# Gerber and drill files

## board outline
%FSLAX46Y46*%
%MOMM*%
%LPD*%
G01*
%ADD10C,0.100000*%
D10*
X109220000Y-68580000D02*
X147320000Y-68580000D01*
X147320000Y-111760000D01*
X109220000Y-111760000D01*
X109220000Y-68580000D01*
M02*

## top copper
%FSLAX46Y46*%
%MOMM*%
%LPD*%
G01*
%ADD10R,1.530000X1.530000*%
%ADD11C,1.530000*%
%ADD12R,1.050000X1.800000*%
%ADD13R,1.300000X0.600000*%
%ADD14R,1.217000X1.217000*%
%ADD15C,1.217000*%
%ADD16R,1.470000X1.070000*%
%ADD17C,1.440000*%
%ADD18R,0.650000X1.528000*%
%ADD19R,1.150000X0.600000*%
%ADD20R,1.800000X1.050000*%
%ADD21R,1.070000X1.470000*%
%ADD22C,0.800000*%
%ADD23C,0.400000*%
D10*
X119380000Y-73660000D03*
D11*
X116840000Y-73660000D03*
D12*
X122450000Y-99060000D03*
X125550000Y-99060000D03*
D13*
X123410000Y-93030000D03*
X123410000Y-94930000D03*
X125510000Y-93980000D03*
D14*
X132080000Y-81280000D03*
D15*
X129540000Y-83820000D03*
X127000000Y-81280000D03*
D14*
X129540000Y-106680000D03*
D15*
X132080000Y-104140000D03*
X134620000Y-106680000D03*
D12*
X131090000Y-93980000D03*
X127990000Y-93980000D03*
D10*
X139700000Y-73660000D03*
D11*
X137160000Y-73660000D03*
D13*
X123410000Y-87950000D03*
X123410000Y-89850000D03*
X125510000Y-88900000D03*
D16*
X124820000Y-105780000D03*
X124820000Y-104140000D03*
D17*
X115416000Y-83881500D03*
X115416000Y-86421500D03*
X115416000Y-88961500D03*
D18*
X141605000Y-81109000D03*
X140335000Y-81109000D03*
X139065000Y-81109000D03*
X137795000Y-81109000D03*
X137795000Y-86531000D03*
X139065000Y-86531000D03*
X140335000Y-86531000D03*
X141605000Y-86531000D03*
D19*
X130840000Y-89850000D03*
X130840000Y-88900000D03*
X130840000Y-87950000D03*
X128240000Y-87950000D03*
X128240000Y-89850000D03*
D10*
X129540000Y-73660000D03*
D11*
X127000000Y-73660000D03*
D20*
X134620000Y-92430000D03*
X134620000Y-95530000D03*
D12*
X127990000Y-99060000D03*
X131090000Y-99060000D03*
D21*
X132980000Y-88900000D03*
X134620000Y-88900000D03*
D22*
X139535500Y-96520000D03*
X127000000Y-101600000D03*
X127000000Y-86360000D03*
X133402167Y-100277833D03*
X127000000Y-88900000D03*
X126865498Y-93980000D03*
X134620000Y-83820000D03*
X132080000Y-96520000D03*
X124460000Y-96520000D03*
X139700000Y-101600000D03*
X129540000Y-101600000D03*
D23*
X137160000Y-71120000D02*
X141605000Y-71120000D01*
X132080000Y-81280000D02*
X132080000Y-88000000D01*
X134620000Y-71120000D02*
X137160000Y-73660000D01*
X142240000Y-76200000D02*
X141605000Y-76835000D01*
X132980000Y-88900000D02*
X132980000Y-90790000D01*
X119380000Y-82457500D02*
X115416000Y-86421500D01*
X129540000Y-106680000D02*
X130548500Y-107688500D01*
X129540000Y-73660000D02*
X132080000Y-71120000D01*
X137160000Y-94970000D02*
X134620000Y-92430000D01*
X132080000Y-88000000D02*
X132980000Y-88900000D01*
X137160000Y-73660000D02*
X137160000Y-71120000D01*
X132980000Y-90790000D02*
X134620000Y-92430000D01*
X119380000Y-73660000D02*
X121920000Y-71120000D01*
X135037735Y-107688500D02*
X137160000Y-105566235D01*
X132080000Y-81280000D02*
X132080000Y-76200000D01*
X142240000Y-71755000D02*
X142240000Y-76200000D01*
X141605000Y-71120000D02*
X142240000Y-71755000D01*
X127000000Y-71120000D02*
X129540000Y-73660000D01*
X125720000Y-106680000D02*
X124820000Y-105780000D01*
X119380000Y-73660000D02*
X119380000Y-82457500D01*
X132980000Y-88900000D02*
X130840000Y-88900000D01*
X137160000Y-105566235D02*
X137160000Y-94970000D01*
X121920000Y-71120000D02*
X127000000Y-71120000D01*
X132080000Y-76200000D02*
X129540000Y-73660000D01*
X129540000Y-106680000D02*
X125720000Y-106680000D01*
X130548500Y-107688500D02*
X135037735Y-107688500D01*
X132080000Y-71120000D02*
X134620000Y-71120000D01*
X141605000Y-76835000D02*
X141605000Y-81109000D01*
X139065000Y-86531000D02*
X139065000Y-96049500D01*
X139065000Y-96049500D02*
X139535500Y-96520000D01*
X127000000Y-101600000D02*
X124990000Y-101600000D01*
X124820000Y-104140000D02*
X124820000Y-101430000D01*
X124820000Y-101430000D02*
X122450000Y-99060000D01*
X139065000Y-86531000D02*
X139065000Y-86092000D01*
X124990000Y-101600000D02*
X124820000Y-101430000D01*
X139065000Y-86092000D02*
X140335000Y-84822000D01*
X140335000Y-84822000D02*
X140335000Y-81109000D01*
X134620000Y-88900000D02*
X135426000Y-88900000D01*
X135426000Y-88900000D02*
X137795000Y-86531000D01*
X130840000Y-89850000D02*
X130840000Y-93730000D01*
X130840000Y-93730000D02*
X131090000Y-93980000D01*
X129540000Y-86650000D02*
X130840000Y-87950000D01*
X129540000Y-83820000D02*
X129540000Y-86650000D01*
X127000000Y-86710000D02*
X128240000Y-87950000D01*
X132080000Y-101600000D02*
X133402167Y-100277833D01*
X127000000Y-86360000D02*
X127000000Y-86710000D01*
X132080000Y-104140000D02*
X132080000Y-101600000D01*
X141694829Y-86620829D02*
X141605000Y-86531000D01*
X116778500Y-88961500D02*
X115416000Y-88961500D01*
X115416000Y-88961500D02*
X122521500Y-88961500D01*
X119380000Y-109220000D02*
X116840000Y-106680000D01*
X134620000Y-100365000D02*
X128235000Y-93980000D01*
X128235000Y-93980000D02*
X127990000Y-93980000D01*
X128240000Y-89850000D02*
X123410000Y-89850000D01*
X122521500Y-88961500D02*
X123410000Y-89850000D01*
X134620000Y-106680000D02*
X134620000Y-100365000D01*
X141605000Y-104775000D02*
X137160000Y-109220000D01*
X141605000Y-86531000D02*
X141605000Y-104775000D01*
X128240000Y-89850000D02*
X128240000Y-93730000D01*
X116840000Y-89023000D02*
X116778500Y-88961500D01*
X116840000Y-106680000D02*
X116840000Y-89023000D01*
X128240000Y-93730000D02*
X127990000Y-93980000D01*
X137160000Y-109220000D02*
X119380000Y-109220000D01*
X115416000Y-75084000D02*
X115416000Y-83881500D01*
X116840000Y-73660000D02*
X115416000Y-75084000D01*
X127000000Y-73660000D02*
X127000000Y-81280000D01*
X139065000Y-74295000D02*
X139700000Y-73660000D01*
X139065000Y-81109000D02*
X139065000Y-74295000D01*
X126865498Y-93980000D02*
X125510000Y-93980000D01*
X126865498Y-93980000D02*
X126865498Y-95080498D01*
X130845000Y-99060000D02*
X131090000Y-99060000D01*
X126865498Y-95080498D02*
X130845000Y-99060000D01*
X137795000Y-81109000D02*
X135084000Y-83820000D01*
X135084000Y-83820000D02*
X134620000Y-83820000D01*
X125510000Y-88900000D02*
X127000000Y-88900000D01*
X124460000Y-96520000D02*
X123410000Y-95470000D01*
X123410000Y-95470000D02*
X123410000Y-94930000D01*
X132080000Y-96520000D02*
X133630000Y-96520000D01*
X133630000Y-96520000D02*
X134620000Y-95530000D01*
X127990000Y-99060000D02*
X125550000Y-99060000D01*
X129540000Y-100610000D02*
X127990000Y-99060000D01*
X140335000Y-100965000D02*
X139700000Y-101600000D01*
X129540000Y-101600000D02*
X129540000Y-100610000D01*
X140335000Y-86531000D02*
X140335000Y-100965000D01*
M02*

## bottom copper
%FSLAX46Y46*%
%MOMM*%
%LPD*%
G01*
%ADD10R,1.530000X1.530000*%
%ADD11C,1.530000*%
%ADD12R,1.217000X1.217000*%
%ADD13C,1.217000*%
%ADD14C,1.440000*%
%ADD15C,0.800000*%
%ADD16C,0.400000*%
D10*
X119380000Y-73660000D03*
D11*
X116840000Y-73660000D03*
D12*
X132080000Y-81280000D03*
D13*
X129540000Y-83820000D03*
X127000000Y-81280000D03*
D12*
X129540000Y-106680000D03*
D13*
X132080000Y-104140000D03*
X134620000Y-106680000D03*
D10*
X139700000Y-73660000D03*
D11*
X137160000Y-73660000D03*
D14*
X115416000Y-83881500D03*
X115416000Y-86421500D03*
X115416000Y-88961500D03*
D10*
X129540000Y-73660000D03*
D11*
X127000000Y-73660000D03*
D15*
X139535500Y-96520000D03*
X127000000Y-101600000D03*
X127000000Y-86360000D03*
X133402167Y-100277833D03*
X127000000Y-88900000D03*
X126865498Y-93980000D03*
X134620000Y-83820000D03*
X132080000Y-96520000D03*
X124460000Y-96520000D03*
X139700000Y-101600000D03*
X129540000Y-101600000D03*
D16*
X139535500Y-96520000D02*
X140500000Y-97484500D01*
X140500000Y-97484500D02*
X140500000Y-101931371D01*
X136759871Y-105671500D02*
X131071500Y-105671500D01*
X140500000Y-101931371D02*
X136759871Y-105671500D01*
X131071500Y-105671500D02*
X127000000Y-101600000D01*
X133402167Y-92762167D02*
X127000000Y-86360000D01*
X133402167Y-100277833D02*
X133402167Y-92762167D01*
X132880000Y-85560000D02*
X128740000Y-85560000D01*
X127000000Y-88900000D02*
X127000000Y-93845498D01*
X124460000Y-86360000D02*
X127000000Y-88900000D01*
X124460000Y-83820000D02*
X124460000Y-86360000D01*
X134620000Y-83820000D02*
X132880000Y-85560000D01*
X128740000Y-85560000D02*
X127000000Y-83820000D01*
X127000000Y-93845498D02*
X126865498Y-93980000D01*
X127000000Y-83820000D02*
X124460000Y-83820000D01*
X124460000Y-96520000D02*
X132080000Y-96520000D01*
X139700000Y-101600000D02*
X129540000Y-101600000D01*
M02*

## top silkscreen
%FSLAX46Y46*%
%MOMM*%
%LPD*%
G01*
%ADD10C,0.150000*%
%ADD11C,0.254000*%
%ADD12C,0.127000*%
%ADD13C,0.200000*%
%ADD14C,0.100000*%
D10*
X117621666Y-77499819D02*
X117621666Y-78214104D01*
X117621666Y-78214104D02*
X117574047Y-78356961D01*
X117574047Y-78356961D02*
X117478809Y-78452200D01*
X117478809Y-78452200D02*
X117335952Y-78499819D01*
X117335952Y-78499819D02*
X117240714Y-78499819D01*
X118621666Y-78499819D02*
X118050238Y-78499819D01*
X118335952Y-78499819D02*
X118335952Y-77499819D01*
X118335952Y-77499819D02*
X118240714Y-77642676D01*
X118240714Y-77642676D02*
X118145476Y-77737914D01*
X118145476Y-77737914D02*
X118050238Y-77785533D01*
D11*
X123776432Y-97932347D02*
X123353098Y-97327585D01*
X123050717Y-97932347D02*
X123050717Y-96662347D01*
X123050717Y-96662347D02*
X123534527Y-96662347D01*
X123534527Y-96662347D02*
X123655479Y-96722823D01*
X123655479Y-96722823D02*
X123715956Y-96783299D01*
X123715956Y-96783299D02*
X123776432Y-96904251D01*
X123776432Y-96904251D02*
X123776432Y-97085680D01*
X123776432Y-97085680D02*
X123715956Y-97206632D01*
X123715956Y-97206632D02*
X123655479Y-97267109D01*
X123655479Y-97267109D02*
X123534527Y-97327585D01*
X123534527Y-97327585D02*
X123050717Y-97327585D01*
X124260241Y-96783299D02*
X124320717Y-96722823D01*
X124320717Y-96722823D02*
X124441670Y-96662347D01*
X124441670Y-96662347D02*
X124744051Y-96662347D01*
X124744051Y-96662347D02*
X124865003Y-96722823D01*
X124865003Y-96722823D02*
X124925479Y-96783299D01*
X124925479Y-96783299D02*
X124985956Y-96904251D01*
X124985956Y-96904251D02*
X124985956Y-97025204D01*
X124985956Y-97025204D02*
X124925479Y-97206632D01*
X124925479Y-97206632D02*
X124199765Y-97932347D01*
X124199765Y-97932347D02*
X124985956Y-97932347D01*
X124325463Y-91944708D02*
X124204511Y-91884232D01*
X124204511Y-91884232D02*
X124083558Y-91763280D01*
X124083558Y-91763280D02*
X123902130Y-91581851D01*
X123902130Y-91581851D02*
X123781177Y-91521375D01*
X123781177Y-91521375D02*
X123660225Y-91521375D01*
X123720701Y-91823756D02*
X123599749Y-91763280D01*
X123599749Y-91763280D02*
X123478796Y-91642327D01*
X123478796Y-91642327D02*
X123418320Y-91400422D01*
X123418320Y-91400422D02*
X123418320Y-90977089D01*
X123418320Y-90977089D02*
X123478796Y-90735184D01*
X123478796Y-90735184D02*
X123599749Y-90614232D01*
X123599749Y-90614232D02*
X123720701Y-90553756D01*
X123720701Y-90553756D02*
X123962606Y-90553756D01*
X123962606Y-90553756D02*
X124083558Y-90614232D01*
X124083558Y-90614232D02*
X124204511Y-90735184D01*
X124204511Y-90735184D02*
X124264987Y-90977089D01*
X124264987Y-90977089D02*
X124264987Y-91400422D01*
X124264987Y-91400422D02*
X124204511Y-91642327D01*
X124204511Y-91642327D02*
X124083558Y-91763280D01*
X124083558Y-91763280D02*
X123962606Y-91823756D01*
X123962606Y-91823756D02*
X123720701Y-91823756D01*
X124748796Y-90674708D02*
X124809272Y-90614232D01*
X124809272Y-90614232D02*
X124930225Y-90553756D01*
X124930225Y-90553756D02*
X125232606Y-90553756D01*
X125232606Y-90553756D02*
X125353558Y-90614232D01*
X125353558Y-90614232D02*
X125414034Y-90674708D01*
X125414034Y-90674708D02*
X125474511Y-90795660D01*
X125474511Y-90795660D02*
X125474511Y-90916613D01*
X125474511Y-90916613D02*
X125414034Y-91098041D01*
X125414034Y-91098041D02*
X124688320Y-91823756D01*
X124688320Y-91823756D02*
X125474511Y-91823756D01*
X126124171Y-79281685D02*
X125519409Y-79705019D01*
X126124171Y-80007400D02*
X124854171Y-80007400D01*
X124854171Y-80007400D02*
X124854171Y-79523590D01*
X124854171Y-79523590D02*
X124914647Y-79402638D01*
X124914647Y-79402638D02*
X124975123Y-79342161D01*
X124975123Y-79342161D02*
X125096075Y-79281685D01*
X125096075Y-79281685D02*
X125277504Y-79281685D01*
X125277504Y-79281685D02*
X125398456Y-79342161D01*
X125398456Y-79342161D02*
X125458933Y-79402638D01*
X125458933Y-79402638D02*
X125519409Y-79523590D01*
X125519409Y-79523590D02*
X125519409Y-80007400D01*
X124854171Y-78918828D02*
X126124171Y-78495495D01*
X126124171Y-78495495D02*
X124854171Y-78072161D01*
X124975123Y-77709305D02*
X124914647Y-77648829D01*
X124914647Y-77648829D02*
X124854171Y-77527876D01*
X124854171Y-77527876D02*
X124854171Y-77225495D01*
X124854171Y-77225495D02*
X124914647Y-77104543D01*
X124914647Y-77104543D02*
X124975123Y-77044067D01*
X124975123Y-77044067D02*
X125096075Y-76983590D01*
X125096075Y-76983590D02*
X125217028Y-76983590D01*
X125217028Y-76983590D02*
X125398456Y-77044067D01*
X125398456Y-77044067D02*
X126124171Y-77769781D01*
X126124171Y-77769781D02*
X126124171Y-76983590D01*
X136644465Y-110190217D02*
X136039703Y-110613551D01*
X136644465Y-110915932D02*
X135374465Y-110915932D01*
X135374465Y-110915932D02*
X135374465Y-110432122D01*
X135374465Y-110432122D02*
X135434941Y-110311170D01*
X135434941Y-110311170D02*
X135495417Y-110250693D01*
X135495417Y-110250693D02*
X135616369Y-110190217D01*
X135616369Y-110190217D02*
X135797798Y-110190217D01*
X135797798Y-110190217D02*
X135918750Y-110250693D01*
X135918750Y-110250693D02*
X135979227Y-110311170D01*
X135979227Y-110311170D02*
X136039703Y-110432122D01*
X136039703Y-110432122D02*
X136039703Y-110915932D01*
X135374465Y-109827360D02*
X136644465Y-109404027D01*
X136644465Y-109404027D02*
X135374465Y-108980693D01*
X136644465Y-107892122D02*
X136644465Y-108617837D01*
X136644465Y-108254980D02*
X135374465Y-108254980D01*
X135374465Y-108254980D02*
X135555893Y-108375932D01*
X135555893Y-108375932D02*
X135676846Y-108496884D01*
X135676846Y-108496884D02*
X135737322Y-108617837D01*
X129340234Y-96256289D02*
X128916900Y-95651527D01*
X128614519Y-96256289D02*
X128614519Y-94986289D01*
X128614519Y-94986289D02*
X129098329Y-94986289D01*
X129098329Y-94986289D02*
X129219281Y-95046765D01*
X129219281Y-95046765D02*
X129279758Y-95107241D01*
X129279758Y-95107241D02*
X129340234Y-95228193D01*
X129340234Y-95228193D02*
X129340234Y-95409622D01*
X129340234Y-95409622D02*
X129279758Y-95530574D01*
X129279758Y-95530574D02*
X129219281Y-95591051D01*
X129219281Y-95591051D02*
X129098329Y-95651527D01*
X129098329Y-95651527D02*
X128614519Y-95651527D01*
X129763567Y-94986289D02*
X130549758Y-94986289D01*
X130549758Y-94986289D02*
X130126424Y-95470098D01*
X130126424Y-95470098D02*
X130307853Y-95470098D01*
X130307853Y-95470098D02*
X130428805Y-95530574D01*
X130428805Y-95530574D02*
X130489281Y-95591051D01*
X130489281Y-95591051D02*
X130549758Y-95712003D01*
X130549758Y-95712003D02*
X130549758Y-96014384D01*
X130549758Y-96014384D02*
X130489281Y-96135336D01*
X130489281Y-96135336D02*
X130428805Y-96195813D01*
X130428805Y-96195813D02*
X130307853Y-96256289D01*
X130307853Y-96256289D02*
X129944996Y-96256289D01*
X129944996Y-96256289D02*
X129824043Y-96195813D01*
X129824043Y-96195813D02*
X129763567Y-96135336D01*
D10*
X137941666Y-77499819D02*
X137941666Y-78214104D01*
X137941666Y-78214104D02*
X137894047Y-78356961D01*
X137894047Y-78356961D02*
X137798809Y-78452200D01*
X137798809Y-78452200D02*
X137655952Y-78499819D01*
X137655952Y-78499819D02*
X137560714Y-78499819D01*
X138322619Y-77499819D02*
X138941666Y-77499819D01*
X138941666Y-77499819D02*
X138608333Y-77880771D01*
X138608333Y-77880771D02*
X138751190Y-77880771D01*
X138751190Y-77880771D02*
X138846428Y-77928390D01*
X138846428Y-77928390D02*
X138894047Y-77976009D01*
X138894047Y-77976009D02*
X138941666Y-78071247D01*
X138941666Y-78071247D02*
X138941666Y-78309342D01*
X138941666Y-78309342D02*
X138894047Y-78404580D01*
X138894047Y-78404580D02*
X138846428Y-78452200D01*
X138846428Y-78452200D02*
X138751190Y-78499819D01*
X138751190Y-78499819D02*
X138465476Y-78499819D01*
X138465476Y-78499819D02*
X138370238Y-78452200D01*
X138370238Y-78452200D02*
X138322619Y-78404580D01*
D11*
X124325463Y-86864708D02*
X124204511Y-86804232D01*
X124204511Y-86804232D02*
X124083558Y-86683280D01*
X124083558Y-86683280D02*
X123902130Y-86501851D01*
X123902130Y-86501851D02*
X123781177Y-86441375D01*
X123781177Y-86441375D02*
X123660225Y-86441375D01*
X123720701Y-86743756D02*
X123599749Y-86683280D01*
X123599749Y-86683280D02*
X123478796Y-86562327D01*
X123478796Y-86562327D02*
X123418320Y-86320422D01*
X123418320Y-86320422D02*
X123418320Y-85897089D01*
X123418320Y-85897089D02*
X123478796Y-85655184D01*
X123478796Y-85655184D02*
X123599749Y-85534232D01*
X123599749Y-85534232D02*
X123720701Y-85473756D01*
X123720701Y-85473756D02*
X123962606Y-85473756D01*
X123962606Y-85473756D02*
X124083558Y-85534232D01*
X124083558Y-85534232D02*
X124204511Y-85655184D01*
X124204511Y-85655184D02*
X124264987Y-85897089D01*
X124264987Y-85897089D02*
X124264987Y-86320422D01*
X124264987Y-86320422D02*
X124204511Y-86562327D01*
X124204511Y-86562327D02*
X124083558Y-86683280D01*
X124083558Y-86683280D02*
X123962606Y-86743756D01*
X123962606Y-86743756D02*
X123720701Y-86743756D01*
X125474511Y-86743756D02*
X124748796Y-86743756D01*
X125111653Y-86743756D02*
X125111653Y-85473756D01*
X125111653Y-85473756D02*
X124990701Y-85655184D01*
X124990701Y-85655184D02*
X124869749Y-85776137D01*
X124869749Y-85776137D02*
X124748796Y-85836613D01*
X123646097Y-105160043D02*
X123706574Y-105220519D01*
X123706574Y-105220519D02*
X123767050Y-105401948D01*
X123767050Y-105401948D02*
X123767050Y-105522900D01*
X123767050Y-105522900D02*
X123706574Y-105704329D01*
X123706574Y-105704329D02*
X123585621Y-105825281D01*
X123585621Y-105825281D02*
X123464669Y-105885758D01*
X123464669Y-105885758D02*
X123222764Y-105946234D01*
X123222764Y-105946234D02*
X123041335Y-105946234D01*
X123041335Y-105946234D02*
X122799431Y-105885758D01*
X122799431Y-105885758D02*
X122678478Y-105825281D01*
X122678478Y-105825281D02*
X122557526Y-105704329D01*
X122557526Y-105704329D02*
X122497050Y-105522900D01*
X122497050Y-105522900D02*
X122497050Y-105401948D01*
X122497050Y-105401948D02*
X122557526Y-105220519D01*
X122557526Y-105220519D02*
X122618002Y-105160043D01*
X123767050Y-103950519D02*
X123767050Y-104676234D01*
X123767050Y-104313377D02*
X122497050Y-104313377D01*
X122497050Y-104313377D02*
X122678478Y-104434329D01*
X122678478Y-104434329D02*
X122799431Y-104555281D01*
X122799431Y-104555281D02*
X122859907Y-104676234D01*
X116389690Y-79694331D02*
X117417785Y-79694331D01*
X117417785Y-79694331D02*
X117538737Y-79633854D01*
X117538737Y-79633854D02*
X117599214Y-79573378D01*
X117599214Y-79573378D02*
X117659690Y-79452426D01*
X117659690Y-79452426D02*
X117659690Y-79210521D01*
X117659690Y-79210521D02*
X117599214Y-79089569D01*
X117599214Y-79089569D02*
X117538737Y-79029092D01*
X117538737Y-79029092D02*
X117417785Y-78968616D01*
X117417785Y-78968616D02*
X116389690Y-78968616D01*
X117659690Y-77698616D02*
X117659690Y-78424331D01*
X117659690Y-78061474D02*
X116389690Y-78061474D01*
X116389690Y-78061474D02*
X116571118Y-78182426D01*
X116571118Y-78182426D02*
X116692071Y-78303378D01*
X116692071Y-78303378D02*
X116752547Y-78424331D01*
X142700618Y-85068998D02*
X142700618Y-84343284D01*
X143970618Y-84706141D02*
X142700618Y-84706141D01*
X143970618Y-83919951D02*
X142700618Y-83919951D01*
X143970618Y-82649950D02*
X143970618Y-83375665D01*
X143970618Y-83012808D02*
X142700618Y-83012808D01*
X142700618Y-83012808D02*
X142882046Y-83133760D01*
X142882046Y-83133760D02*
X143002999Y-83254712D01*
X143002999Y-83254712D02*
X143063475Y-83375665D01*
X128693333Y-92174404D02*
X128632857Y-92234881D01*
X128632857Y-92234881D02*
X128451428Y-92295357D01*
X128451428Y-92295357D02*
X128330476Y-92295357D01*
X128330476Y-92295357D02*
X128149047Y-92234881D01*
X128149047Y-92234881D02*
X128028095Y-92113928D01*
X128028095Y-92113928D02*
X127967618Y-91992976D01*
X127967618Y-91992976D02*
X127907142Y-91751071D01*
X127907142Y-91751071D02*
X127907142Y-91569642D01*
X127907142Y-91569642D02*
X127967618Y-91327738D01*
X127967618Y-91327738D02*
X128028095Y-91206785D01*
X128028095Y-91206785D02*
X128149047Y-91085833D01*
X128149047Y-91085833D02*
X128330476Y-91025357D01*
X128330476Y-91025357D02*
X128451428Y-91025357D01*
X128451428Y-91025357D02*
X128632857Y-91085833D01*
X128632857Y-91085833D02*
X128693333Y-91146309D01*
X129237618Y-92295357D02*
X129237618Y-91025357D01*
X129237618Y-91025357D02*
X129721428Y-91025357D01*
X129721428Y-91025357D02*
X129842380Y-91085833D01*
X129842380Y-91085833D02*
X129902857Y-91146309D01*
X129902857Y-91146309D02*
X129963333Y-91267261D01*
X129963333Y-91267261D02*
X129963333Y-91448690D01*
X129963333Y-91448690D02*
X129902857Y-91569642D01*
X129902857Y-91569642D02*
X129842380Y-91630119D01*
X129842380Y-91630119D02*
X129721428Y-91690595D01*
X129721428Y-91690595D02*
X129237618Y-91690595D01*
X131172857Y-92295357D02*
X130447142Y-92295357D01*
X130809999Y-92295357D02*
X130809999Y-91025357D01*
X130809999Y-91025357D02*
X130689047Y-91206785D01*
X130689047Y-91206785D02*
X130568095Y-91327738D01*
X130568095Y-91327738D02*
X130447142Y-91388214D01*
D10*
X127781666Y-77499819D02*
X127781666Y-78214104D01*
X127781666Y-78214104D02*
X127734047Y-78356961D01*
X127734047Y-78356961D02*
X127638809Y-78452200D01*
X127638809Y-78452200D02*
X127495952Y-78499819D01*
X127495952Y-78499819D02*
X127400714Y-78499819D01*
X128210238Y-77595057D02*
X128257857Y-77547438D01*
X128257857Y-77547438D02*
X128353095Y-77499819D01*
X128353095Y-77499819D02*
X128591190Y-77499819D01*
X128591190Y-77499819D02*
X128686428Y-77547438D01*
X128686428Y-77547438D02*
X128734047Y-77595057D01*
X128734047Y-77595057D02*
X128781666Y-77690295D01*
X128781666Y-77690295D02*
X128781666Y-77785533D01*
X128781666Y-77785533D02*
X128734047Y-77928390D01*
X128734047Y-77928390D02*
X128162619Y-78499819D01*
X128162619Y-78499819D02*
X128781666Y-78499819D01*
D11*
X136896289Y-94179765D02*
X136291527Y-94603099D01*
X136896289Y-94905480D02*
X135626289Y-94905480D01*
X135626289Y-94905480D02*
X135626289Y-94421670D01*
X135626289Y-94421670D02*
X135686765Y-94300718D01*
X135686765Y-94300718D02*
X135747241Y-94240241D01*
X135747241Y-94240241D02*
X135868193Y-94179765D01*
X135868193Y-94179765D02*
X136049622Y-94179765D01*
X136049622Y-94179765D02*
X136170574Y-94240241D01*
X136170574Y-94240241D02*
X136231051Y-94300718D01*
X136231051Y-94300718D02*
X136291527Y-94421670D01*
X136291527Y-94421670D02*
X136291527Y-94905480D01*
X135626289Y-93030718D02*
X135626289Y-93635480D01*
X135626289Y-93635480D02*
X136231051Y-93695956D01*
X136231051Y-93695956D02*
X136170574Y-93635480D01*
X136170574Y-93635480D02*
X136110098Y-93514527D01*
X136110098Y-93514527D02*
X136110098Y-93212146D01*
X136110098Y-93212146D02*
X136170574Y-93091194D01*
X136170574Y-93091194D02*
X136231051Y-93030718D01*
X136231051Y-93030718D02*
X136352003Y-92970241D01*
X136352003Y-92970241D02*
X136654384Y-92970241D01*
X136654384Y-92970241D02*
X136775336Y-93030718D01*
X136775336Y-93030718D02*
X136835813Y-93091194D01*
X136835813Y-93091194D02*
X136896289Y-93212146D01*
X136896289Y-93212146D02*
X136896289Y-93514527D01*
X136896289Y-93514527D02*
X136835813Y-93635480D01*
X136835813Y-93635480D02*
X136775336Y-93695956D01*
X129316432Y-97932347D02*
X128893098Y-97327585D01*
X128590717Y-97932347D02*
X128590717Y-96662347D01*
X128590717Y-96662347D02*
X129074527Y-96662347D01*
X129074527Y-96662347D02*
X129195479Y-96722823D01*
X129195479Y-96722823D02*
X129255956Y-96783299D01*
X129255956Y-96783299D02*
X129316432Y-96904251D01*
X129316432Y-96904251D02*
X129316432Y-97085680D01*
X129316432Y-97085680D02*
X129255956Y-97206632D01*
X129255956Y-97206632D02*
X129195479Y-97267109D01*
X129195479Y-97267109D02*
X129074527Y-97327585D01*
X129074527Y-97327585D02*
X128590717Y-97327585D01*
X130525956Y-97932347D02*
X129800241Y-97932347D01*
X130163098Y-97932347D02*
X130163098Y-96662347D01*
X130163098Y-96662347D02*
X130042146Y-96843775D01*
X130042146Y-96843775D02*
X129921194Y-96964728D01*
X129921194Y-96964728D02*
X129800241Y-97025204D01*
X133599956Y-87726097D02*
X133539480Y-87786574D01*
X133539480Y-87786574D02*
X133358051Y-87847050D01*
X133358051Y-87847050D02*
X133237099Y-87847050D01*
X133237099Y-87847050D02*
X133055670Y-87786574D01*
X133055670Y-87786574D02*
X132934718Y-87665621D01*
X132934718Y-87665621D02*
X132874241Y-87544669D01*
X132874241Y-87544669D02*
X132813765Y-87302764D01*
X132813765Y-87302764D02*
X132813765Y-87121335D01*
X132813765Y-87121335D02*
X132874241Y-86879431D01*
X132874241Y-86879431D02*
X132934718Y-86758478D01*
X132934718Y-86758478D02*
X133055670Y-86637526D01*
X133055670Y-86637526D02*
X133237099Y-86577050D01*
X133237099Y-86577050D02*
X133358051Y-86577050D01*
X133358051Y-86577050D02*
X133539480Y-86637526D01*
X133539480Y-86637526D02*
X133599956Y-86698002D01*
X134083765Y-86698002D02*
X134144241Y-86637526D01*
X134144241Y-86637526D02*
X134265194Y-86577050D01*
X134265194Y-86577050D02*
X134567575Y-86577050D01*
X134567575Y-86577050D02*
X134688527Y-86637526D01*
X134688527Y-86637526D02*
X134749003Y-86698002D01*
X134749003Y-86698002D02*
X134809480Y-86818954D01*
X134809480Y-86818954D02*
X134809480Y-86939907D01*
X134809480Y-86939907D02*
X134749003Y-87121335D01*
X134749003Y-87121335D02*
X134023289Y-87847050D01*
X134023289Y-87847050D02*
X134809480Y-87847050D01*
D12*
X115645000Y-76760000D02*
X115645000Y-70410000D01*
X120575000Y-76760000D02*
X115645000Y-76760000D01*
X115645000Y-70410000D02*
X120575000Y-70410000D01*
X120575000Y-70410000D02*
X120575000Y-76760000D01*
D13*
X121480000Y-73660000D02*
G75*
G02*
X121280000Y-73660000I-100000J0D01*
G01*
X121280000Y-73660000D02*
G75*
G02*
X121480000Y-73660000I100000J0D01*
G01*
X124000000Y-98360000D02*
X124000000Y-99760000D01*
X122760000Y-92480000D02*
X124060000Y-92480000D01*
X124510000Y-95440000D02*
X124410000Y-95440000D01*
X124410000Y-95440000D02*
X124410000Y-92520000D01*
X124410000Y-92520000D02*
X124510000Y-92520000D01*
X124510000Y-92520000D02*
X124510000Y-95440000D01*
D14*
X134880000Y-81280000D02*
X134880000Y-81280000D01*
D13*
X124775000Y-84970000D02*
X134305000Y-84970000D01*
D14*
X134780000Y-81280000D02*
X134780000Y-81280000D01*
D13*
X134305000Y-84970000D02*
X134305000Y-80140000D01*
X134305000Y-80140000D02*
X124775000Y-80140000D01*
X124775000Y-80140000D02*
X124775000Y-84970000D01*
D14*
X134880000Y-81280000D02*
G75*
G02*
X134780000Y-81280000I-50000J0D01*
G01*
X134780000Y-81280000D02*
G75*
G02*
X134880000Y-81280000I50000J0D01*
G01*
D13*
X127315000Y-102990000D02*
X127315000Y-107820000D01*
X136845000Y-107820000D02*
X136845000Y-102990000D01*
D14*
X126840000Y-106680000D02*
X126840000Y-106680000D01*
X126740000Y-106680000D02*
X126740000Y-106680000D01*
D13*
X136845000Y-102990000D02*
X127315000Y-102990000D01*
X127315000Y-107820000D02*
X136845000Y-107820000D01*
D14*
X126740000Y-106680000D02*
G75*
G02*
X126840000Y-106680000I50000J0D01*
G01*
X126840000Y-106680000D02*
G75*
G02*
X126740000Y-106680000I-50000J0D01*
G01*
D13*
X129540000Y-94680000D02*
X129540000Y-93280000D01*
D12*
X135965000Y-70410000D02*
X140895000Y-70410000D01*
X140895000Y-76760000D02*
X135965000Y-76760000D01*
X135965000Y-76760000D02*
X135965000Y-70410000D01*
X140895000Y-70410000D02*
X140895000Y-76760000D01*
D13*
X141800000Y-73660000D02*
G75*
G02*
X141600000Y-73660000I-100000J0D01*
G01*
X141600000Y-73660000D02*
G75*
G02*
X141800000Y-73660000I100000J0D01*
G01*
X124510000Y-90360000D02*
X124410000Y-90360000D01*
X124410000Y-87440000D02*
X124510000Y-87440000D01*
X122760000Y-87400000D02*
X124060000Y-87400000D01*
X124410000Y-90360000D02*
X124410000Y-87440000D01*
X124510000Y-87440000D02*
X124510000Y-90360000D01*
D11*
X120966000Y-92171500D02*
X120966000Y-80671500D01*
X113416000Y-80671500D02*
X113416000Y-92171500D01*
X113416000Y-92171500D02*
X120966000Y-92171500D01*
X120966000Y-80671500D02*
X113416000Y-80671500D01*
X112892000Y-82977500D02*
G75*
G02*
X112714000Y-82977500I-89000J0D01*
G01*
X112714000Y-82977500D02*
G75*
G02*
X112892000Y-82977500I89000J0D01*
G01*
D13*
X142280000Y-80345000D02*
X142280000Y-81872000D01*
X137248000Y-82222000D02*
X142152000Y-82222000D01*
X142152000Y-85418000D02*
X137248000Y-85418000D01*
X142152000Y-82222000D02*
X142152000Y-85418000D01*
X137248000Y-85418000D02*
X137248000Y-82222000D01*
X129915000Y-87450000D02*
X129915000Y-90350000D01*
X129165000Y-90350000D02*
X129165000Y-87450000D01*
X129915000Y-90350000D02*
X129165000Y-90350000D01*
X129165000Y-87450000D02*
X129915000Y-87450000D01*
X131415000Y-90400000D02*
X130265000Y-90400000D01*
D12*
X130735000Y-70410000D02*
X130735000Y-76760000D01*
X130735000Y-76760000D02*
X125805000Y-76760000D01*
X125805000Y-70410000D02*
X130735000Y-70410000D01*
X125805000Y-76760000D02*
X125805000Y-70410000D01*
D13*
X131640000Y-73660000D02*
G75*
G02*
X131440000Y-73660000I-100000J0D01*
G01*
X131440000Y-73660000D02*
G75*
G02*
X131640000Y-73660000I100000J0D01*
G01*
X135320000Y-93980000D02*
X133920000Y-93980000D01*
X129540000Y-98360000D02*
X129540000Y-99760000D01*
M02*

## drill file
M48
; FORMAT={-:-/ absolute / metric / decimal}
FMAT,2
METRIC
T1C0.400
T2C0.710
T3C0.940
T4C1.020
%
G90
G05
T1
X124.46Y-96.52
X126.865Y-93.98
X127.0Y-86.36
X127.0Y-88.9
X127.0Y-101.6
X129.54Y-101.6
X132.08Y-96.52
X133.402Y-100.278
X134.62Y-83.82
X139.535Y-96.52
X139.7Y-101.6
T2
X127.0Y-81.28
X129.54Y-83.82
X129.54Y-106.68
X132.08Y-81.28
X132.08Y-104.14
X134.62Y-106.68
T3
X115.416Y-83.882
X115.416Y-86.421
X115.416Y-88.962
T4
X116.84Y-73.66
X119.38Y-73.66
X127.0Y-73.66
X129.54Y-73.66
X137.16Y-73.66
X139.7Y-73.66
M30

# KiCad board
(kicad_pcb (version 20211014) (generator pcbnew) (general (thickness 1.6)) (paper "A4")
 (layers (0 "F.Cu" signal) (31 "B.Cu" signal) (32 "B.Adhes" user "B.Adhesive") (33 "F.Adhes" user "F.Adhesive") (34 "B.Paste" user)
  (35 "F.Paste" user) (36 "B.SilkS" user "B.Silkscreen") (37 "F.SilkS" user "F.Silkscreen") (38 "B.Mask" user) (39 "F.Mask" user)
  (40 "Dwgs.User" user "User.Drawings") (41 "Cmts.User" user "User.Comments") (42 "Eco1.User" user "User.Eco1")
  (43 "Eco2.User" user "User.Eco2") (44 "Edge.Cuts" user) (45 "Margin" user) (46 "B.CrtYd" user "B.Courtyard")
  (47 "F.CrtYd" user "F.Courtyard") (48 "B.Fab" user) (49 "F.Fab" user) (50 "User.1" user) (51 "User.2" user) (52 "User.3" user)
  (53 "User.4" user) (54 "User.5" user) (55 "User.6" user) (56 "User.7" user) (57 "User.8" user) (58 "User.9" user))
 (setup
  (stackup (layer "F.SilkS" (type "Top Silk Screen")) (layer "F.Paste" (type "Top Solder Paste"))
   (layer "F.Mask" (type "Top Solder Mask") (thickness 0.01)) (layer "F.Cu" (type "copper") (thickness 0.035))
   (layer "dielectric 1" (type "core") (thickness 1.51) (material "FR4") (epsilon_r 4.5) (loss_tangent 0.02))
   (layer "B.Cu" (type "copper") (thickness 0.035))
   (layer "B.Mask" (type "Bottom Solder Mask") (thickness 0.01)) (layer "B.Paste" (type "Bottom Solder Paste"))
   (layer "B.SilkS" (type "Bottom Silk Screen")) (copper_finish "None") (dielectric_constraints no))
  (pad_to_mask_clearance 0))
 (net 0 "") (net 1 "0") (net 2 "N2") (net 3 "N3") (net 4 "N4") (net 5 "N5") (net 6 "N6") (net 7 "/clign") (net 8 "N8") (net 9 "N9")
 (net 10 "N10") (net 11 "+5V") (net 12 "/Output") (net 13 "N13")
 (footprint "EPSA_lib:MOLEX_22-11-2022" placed (layer "F.Cu") (at 119.38 73.66 180)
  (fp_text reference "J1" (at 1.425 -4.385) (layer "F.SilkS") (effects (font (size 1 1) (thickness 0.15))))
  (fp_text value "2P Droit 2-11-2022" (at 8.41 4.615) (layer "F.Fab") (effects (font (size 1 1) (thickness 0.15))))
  (fp_line (start 3.735 -3.1) (end 3.735 3.25) (layer "F.SilkS") (width 0.127))
  (fp_line (start -1.195 -3.1) (end 3.735 -3.1) (layer "F.SilkS") (width 0.127))
  (fp_line (start 3.735 3.25) (end -1.195 3.25) (layer "F.SilkS") (width 0.127))
  (fp_line (start -1.195 3.25) (end -1.195 -3.1) (layer "F.SilkS") (width 0.127))
  (fp_circle (center -2 0) (end -1.9 0) (layer "F.SilkS") (width 0.2) (fill none))
  (pad "1" thru_hole rect (at 0 0 180) (size 1.53 1.53) (drill 1.02) (layers *.Cu *.Mask) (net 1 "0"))
  (pad "2" thru_hole circle (at 2.54 0 180) (size 1.53 1.53) (drill 1.02) (layers *.Cu *.Mask) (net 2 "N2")))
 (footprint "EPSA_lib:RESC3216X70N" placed (layer "F.Cu") (at 124 99.06)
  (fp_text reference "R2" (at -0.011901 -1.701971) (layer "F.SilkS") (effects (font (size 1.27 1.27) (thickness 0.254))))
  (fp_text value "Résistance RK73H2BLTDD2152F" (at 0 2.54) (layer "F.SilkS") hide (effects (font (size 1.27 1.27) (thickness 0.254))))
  (fp_line (start 0 -0.7) (end 0 0.7) (layer "F.SilkS") (width 0.2))
  (pad "1" smd rect (at -1.55 0) (size 1.05 1.8) (layers "F.Cu" "F.Paste" "F.Mask") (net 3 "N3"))
  (pad "2" smd rect (at 1.55 0) (size 1.05 1.8) (layers "F.Cu" "F.Paste" "F.Mask") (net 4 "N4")))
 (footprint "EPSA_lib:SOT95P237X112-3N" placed (layer "F.Cu") (at 124.46 93.98)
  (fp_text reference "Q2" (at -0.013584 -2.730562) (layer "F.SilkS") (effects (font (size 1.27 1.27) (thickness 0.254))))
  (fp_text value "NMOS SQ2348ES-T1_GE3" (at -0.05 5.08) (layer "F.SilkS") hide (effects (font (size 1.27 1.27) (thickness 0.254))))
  (fp_line (start -1.7 -1.5) (end -0.4 -1.5) (layer "F.SilkS") (width 0.2))
  (fp_line (start 0.05 1.46) (end -0.05 1.46) (layer "F.SilkS") (width 0.2))
  (fp_line (start -0.05 1.46) (end -0.05 -1.46) (layer "F.SilkS") (width 0.2))
  (fp_line (start -0.05 -1.46) (end 0.05 -1.46) (layer "F.SilkS") (width 0.2))
  (fp_line (start 0.05 -1.46) (end 0.05 1.46) (layer "F.SilkS") (width 0.2))
  (pad "1" smd rect (at -1.05 -0.95 90) (size 0.6 1.3) (layers "F.Cu" "F.Paste" "F.Mask") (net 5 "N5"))
  (pad "2" smd rect (at -1.05 0.95 90) (size 0.6 1.3) (layers "F.Cu" "F.Paste" "F.Mask") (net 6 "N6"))
  (pad "3" smd rect (at 1.05 0 90) (size 0.6 1.3) (layers "F.Cu" "F.Paste" "F.Mask") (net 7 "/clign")))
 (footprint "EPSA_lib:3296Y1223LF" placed (layer "F.Cu") (at 132.08 81.28 90)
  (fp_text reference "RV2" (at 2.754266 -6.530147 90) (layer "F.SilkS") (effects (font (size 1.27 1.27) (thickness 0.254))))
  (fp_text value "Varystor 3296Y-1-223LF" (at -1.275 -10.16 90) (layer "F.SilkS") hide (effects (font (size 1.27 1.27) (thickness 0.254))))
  (fp_line (start 0 2.8) (end 0 2.8) (layer "F.SilkS") (width 0.1))
  (fp_line (start -3.69 -7.305) (end -3.69 2.225) (layer "F.SilkS") (width 0.2))
  (fp_line (start 0 2.7) (end 0 2.7) (layer "F.SilkS") (width 0.1))
  (fp_line (start -3.69 2.225) (end 1.14 2.225) (layer "F.SilkS") (width 0.2))
  (fp_line (start 1.14 2.225) (end 1.14 -7.305) (layer "F.SilkS") (width 0.2))
  (fp_line (start 1.14 -7.305) (end -3.69 -7.305) (layer "F.SilkS") (width 0.2))
  (fp_arc (start 0 2.8) (mid -0.05 2.75) (end 0 2.7) (layer "F.SilkS") (width 0.1))
  (fp_arc (start 0 2.7) (mid 0.05 2.75) (end 0 2.8) (layer "F.SilkS") (width 0.1))
  (pad "1" thru_hole rect (at 0 0 90) (size 1.217 1.217) (drill 0.71) (layers *.Cu *.Mask) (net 1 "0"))
  (pad "2" thru_hole circle (at -2.54 -2.54 90) (size 1.217 1.217) (drill 0.71) (layers *.Cu *.Mask) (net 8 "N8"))
  (pad "3" thru_hole circle (at 0 -5.08 90) (size 1.217 1.217) (drill 0.71) (layers *.Cu *.Mask) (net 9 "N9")))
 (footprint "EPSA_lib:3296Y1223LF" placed (layer "F.Cu") (at 129.54 106.68 -90)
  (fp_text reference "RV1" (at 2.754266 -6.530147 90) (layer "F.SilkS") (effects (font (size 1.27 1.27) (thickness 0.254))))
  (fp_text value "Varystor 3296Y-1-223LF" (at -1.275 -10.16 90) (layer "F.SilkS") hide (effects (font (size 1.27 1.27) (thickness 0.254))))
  (fp_line (start -3.69 2.225) (end 1.14 2.225) (layer "F.SilkS") (width 0.2))
  (fp_line (start 1.14 -7.305) (end -3.69 -7.305) (layer "F.SilkS") (width 0.2))
  (fp_line (start 0 2.7) (end 0 2.7) (layer "F.SilkS") (width 0.1))
  (fp_line (start 0 2.8) (end 0 2.8) (layer "F.SilkS") (width 0.1))
  (fp_line (start -3.69 -7.305) (end -3.69 2.225) (layer "F.SilkS") (width 0.2))
  (fp_line (start 1.14 2.225) (end 1.14 -7.305) (layer "F.SilkS") (width 0.2))
  (fp_arc (start 0 2.8) (mid -0.05 2.75) (end 0 2.7) (layer "F.SilkS") (width 0.1))
  (fp_arc (start 0 2.7) (mid 0.05 2.75) (end 0 2.8) (layer "F.SilkS") (width 0.1))
  (pad "1" thru_hole rect (at 0 0 270) (size 1.217 1.217) (drill 0.71) (layers *.Cu *.Mask) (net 1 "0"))
  (pad "2" thru_hole circle (at -2.54 -2.54 270) (size 1.217 1.217) (drill 0.71) (layers *.Cu *.Mask) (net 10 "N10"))
  (pad "3" thru_hole circle (at 0 -5.08 270) (size 1.217 1.217) (drill 0.71) (layers *.Cu *.Mask) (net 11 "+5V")))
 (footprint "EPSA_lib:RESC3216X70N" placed (layer "F.Cu") (at 129.54 93.98 180)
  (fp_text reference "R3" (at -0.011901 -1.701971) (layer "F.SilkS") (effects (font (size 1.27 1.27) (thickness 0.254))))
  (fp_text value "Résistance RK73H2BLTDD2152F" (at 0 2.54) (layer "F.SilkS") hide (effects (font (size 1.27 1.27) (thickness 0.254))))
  (fp_line (start 0 -0.7) (end 0 0.7) (layer "F.SilkS") (width 0.2))
  (pad "1" smd rect (at -1.55 0 180) (size 1.05 1.8) (layers "F.Cu" "F.Paste" "F.Mask") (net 5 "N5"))
  (pad "2" smd rect (at 1.55 0 180) (size 1.05 1.8) (layers "F.Cu" "F.Paste" "F.Mask") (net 11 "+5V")))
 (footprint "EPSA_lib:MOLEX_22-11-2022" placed (layer "F.Cu") (at 139.7 73.66 180)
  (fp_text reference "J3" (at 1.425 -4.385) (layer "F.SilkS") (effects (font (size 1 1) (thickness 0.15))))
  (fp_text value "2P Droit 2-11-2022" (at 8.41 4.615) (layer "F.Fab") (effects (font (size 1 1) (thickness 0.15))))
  (fp_line (start 3.735 3.25) (end -1.195 3.25) (layer "F.SilkS") (width 0.127))
  (fp_line (start -1.195 -3.1) (end 3.735 -3.1) (layer "F.SilkS") (width 0.127))
  (fp_line (start 3.735 -3.1) (end 3.735 3.25) (layer "F.SilkS") (width 0.127))
  (fp_line (start -1.195 3.25) (end -1.195 -3.1) (layer "F.SilkS") (width 0.127))
  (fp_circle (center -2 0) (end -1.9 0) (layer "F.SilkS") (width 0.2) (fill none))
  (pad "1" thru_hole rect (at 0 0 180) (size 1.53 1.53) (drill 1.02) (layers *.Cu *.Mask) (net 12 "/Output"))
  (pad "2" thru_hole circle (at 2.54 0 180) (size 1.53 1.53) (drill 1.02) (layers *.Cu *.Mask) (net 1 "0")))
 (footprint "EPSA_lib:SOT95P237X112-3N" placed (layer "F.Cu") (at 124.46 88.9)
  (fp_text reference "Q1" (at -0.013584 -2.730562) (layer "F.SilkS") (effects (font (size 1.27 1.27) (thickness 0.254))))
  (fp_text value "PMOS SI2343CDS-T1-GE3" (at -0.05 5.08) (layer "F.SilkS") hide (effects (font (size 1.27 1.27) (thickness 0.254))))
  (fp_line (start 0.05 1.46) (end -0.05 1.46) (layer "F.SilkS") (width 0.2))
  (fp_line (start -0.05 -1.46) (end 0.05 -1.46) (layer "F.SilkS") (width 0.2))
  (fp_line (start -1.7 -1.5) (end -0.4 -1.5) (layer "F.SilkS") (width 0.2))
  (fp_line (start -0.05 1.46) (end -0.05 -1.46) (layer "F.SilkS") (width 0.2))
  (fp_line (start 0.05 -1.46) (end 0.05 1.46) (layer "F.SilkS") (width 0.2))
  (pad "1" smd rect (at -1.05 -0.95 90) (size 0.6 1.3) (layers "F.Cu" "F.Paste" "F.Mask") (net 5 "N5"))
  (pad "2" smd rect (at -1.05 0.95 90) (size 0.6 1.3) (layers "F.Cu" "F.Paste" "F.Mask") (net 11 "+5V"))
  (pad "3" smd rect (at 1.05 0 90) (size 0.6 1.3) (layers "F.Cu" "F.Paste" "F.Mask") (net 7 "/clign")))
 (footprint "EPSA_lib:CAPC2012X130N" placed (layer "F.Cu") (at 124.82 104.96 90)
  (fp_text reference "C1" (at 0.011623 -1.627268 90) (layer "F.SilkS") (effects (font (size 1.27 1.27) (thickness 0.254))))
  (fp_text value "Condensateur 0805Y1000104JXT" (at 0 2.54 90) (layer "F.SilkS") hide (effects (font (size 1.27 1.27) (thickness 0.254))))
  (pad "1" smd rect (at -0.82 0 90) (size 1.07 1.47) (layers "F.Cu" "F.Paste" "F.Mask") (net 1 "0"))
  (pad "2" smd rect (at 0.82 0 90) (size 1.07 1.47) (layers "F.Cu" "F.Paste" "F.Mask") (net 3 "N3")))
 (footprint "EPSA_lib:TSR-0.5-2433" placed (layer "F.Cu") (at 113.416 80.6715 -90)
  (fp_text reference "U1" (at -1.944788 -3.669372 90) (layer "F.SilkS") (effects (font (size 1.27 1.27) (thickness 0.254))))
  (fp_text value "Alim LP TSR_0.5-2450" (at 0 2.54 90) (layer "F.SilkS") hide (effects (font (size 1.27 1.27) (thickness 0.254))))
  (fp_line (start 11.5 -7.55) (end 0 -7.55) (layer "F.SilkS") (width 0.254))
  (fp_line (start 0 0) (end 11.5 0) (layer "F.SilkS") (width 0.254))
  (fp_line (start 11.5 0) (end 11.5 -7.55) (layer "F.SilkS") (width 0.254))
  (fp_line (start 0 -7.55) (end 0 0) (layer "F.SilkS") (width 0.254))
  (fp_circle (center 2.306 0.613) (end 2.306 0.702) (layer "F.SilkS") (width 0.254) (fill none))
  (pad "1" thru_hole circle (at 3.21 -2 270) (size 1.44 1.44) (drill 0.94) (layers *.Cu *.Mask) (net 2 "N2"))
  (pad "2" thru_hole circle (at 5.75 -2 270) (size 1.44 1.44) (drill 0.94) (layers *.Cu *.Mask) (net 1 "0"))
  (pad "3" thru_hole circle (at 8.29 -2 270) (size 1.44 1.44) (drill 0.94) (layers *.Cu *.Mask) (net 11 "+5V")))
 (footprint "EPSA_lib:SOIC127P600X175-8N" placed (layer "F.Cu") (at 139.7 83.82 -90)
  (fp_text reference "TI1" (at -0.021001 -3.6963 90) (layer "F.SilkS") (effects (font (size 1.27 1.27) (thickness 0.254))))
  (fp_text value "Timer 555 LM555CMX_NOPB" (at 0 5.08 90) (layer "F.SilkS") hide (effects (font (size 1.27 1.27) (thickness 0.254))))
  (fp_line (start -3.475 -2.58) (end -1.948 -2.58) (layer "F.SilkS") (width 0.2))
  (fp_line (start -1.598 2.452) (end -1.598 -2.452) (layer "F.SilkS") (width 0.2))
  (fp_line (start 1.598 -2.452) (end 1.598 2.452) (layer "F.SilkS") (width 0.2))
  (fp_line (start -1.598 -2.452) (end 1.598 -2.452) (layer "F.SilkS") (width 0.2))
  (fp_line (start 1.598 2.452) (end -1.598 2.452) (layer "F.SilkS") (width 0.2))
  (pad "1" smd rect (at -2.711 -1.905) (size 0.65 1.528) (layers "F.Cu" "F.Paste" "F.Mask") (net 1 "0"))
  (pad "2" smd rect (at -2.711 -0.635) (size 0.65 1.528) (layers "F.Cu" "F.Paste" "F.Mask") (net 3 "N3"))
  (pad "3" smd rect (at -2.711 0.635) (size 0.65 1.528) (layers "F.Cu" "F.Paste" "F.Mask") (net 12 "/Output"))
  (pad "4" smd rect (at -2.711 1.905) (size 0.65 1.528) (layers "F.Cu" "F.Paste" "F.Mask") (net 7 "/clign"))
  (pad "5" smd rect (at 2.711 1.905) (size 0.65 1.528) (layers "F.Cu" "F.Paste" "F.Mask") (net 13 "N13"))
  (pad "6" smd rect (at 2.711 0.635) (size 0.65 1.528) (layers "F.Cu" "F.Paste" "F.Mask") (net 3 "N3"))
  (pad "7" smd rect (at 2.711 -0.635) (size 0.65 1.528) (layers "F.Cu" "F.Paste" "F.Mask") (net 4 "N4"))
  (pad "8" smd rect (at 2.711 -1.905) (size 0.65 1.528) (layers "F.Cu" "F.Paste" "F.Mask") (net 11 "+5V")))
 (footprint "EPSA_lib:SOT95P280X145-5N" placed (layer "F.Cu") (at 129.54 88.9 180)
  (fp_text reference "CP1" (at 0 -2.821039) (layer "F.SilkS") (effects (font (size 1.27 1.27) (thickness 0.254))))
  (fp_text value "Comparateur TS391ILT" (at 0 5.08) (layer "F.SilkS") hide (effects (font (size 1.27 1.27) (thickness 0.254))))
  (fp_line (start -0.375 1.45) (end -0.375 -1.45) (layer "F.SilkS") (width 0.2))
  (fp_line (start 0.375 -1.45) (end 0.375 1.45) (layer "F.SilkS") (width 0.2))
  (fp_line (start -0.375 -1.45) (end 0.375 -1.45) (layer "F.SilkS") (width 0.2))
  (fp_line (start 0.375 1.45) (end -0.375 1.45) (layer "F.SilkS") (width 0.2))
  (fp_line (start -1.875 -1.5) (end -0.725 -1.5) (layer "F.SilkS") (width 0.2))
  (pad "1" smd rect (at -1.3 -0.95 270) (size 0.6 1.15) (layers "F.Cu" "F.Paste" "F.Mask") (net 5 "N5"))
  (pad "2" smd rect (at -1.3 0 270) (size 0.6 1.15) (layers "F.Cu" "F.Paste" "F.Mask") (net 1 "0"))
  (pad "3" smd rect (at -1.3 0.95 270) (size 0.6 1.15) (layers "F.Cu" "F.Paste" "F.Mask") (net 8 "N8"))
  (pad "4" smd rect (at 1.3 0.95 270) (size 0.6 1.15) (layers "F.Cu" "F.Paste" "F.Mask") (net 10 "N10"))
  (pad "5" smd rect (at 1.3 -0.95 270) (size 0.6 1.15) (layers "F.Cu" "F.Paste" "F.Mask") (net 11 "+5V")))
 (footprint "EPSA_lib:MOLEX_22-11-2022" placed (layer "F.Cu") (at 129.54 73.66 180)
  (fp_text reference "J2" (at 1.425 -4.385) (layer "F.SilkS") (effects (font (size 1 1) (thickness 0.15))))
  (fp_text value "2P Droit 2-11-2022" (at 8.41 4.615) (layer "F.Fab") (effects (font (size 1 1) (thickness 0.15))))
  (fp_line (start -1.195 3.25) (end -1.195 -3.1) (layer "F.SilkS") (width 0.127))
  (fp_line (start -1.195 -3.1) (end 3.735 -3.1) (layer "F.SilkS") (width 0.127))
  (fp_line (start 3.735 3.25) (end -1.195 3.25) (layer "F.SilkS") (width 0.127))
  (fp_line (start 3.735 -3.1) (end 3.735 3.25) (layer "F.SilkS") (width 0.127))
  (fp_circle (center -2 0) (end -1.9 0) (layer "F.SilkS") (width 0.2) (fill none))
  (pad "1" thru_hole rect (at 0 0 180) (size 1.53 1.53) (drill 1.02) (layers *.Cu *.Mask) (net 1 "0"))
  (pad "2" thru_hole circle (at 2.54 0 180) (size 1.53 1.53) (drill 1.02) (layers *.Cu *.Mask) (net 9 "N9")))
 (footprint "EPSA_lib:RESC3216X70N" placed (layer "F.Cu") (at 134.62 93.98 -90)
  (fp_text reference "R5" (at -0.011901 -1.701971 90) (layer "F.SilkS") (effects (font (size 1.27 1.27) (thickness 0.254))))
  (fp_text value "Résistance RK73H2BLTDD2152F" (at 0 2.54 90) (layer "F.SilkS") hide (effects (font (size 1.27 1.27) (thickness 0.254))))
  (fp_line (start 0 -0.7) (end 0 0.7) (layer "F.SilkS") (width 0.2))
  (pad "1" smd rect (at -1.55 0 270) (size 1.05 1.8) (layers "F.Cu" "F.Paste" "F.Mask") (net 1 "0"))
  (pad "2" smd rect (at 1.55 0 270) (size 1.05 1.8) (layers "F.Cu" "F.Paste" "F.Mask") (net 6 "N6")))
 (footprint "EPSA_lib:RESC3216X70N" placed (layer "F.Cu") (at 129.54 99.06)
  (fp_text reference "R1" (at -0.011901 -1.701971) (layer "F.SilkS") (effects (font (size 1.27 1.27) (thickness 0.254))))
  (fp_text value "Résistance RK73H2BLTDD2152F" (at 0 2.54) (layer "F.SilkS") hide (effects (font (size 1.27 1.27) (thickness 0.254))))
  (fp_line (start 0 -0.7) (end 0 0.7) (layer "F.SilkS") (width 0.2))
  (pad "1" smd rect (at -1.55 0) (size 1.05 1.8) (layers "F.Cu" "F.Paste" "F.Mask") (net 4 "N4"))
  (pad "2" smd rect (at 1.55 0) (size 1.05 1.8) (layers "F.Cu" "F.Paste" "F.Mask") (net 7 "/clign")))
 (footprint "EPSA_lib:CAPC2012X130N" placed (layer "F.Cu") (at 133.8 88.9)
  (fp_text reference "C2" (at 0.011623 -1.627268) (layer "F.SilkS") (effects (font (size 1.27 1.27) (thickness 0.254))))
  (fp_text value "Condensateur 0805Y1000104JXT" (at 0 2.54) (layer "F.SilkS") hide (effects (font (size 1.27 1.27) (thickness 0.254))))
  (pad "1" smd rect (at -0.82 0) (size 1.07 1.47) (layers "F.Cu" "F.Paste" "F.Mask") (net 1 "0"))
  (pad "2" smd rect (at 0.82 0) (size 1.07 1.47) (layers "F.Cu" "F.Paste" "F.Mask") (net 13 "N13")))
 (gr_rect (start 147.32 111.76) (end 109.22 68.58) (layer "Edge.Cuts") (width 0.1) (fill none))
 (segment (start 137.16 71.12) (end 141.605 71.12) (width 0.4) (layer "F.Cu") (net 1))
 (segment (start 132.08 81.28) (end 132.08 88) (width 0.4) (layer "F.Cu") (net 1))
 (segment (start 134.62 71.12) (end 137.16 73.66) (width 0.4) (layer "F.Cu") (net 1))
 (segment (start 142.24 76.2) (end 141.605 76.835) (width 0.4) (layer "F.Cu") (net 1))
 (segment (start 132.98 88.9) (end 132.98 90.79) (width 0.4) (layer "F.Cu") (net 1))
 (segment (start 119.38 82.4575) (end 115.416 86.4215) (width 0.4) (layer "F.Cu") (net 1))
 (segment (start 129.54 106.68) (end 130.5485 107.6885) (width 0.4) (layer "F.Cu") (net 1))
 (segment (start 129.54 73.66) (end 132.08 71.12) (width 0.4) (layer "F.Cu") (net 1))
 (segment (start 137.16 94.97) (end 134.62 92.43) (width 0.4) (layer "F.Cu") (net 1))
 (segment (start 132.08 88) (end 132.98 88.9) (width 0.4) (layer "F.Cu") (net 1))
 (segment (start 137.16 73.66) (end 137.16 71.12) (width 0.4) (layer "F.Cu") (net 1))
 (segment (start 132.98 90.79) (end 134.62 92.43) (width 0.4) (layer "F.Cu") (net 1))
 (segment (start 119.38 73.66) (end 121.92 71.12) (width 0.4) (layer "F.Cu") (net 1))
 (segment (start 135.037735 107.6885) (end 137.16 105.566235) (width 0.4) (layer "F.Cu") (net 1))
 (segment (start 132.08 81.28) (end 132.08 76.2) (width 0.4) (layer "F.Cu") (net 1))
 (segment (start 142.24 71.755) (end 142.24 76.2) (width 0.4) (layer "F.Cu") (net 1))
 (segment (start 141.605 71.12) (end 142.24 71.755) (width 0.4) (layer "F.Cu") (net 1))
 (segment (start 127 71.12) (end 129.54 73.66) (width 0.4) (layer "F.Cu") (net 1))
 (segment (start 125.72 106.68) (end 124.82 105.78) (width 0.4) (layer "F.Cu") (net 1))
 (segment (start 119.38 73.66) (end 119.38 82.4575) (width 0.4) (layer "F.Cu") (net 1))
 (segment (start 132.98 88.9) (end 130.84 88.9) (width 0.4) (layer "F.Cu") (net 1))
 (segment (start 137.16 105.566235) (end 137.16 94.97) (width 0.4) (layer "F.Cu") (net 1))
 (segment (start 121.92 71.12) (end 127 71.12) (width 0.4) (layer "F.Cu") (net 1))
 (segment (start 132.08 76.2) (end 129.54 73.66) (width 0.4) (layer "F.Cu") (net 1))
 (segment (start 129.54 106.68) (end 125.72 106.68) (width 0.4) (layer "F.Cu") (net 1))
 (segment (start 130.5485 107.6885) (end 135.037735 107.6885) (width 0.4) (layer "F.Cu") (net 1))
 (segment (start 132.08 71.12) (end 134.62 71.12) (width 0.4) (layer "F.Cu") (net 1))
 (segment (start 141.605 76.835) (end 141.605 81.109) (width 0.4) (layer "F.Cu") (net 1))
 (segment (start 139.065 86.531) (end 139.065 96.0495) (width 0.4) (layer "F.Cu") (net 3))
 (segment (start 139.065 96.0495) (end 139.5355 96.52) (width 0.4) (layer "F.Cu") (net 3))
 (segment (start 127 101.6) (end 124.99 101.6) (width 0.4) (layer "F.Cu") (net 3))
 (segment (start 124.82 104.14) (end 124.82 101.43) (width 0.4) (layer "F.Cu") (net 3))
 (segment (start 124.82 101.43) (end 122.45 99.06) (width 0.4) (layer "F.Cu") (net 3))
 (segment (start 139.065 86.531) (end 139.065 86.092) (width 0.4) (layer "F.Cu") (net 3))
 (segment (start 124.99 101.6) (end 124.82 101.43) (width 0.4) (layer "F.Cu") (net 3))
 (segment (start 139.065 86.092) (end 140.335 84.822) (width 0.4) (layer "F.Cu") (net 3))
 (segment (start 140.335 84.822) (end 140.335 81.109) (width 0.4) (layer "F.Cu") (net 3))
 (via (at 139.5355 96.52) (size 0.8) (drill 0.4) (layers "F.Cu" "B.Cu") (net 3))
 (via (at 127 101.6) (size 0.8) (drill 0.4) (layers "F.Cu" "B.Cu") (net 3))
 (segment (start 139.5355 96.52) (end 140.5 97.4845) (width 0.4) (layer "B.Cu") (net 3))
 (segment (start 140.5 97.4845) (end 140.5 101.931371) (width 0.4) (layer "B.Cu") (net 3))
 (segment (start 136.759871 105.6715) (end 131.0715 105.6715) (width 0.4) (layer "B.Cu") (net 3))
 (segment (start 140.5 101.931371) (end 136.759871 105.6715) (width 0.4) (layer "B.Cu") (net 3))
 (segment (start 131.0715 105.6715) (end 127 101.6) (width 0.4) (layer "B.Cu") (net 3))
 (segment (start 134.62 88.9) (end 135.426 88.9) (width 0.4) (layer "F.Cu") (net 13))
 (segment (start 135.426 88.9) (end 137.795 86.531) (width 0.4) (layer "F.Cu") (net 13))
 (segment (start 130.84 89.85) (end 130.84 93.73) (width 0.4) (layer "F.Cu") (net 5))
 (segment (start 130.84 93.73) (end 131.09 93.98) (width 0.4) (layer "F.Cu") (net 5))
 (segment (start 129.54 86.65) (end 130.84 87.95) (width 0.4) (layer "F.Cu") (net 8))
 (segment (start 129.54 83.82) (end 129.54 86.65) (width 0.4) (layer "F.Cu") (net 8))
 (segment (start 127 86.71) (end 128.24 87.95) (width 0.4) (layer "F.Cu") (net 10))
 (segment (start 132.08 101.6) (end 133.402167 100.277833) (width 0.4) (layer "F.Cu") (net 10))
 (segment (start 127 86.36) (end 127 86.71) (width 0.4) (layer "F.Cu") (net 10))
 (segment (start 132.08 104.14) (end 132.08 101.6) (width 0.4) (layer "F.Cu") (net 10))
 (via (at 127 86.36) (size 0.8) (drill 0.4) (layers "F.Cu" "B.Cu") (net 10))
 (via (at 133.402167 100.277833) (size 0.8) (drill 0.4) (layers "F.Cu" "B.Cu") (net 10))
 (segment (start 133.402167 92.762167) (end 127 86.36) (width 0.4) (layer "B.Cu") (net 10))
 (segment (start 133.402167 100.277833) (end 133.402167 92.762167) (width 0.4) (layer "B.Cu") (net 10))
 (segment (start 141.694829 86.620829) (end 141.605 86.531) (width 0.4) (layer "F.Cu") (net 11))
 (segment (start 116.7785 88.9615) (end 115.416 88.9615) (width 0.4) (layer "F.Cu") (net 11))
 (segment (start 115.416 88.9615) (end 122.5215 88.9615) (width 0.4) (layer "F.Cu") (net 11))
 (segment (start 119.38 109.22) (end 116.84 106.68) (width 0.4) (layer "F.Cu") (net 11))
 (segment (start 134.62 100.365) (end 128.235 93.98) (width 0.4) (layer "F.Cu") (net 11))
 (segment (start 128.235 93.98) (end 127.99 93.98) (width 0.4) (layer "F.Cu") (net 11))
 (segment (start 128.24 89.85) (end 123.41 89.85) (width 0.4) (layer "F.Cu") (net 11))
 (segment (start 122.5215 88.9615) (end 123.41 89.85) (width 0.4) (layer "F.Cu") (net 11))
 (segment (start 134.62 106.68) (end 134.62 100.365) (width 0.4) (layer "F.Cu") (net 11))
 (segment (start 141.605 104.775) (end 137.16 109.22) (width 0.4) (layer "F.Cu") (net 11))
 (segment (start 141.605 86.531) (end 141.605 104.775) (width 0.4) (layer "F.Cu") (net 11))
 (segment (start 128.24 89.85) (end 128.24 93.73) (width 0.4) (layer "F.Cu") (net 11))
 (segment (start 116.84 89.023) (end 116.7785 88.9615) (width 0.4) (layer "F.Cu") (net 11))
 (segment (start 116.84 106.68) (end 116.84 89.023) (width 0.4) (layer "F.Cu") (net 11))
 (segment (start 128.24 93.73) (end 127.99 93.98) (width 0.4) (layer "F.Cu") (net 11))
 (segment (start 137.16 109.22) (end 119.38 109.22) (width 0.4) (layer "F.Cu") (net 11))
 (segment (start 115.416 75.084) (end 115.416 83.8815) (width 0.4) (layer "F.Cu") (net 2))
 (segment (start 116.84 73.66) (end 115.416 75.084) (width 0.4) (layer "F.Cu") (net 2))
 (segment (start 127 73.66) (end 127 81.28) (width 0.4) (layer "F.Cu") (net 9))
 (segment (start 139.065 74.295) (end 139.7 73.66) (width 0.4) (layer "F.Cu") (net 12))
 (segment (start 139.065 81.109) (end 139.065 74.295) (width 0.4) (layer "F.Cu") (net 12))
 (segment (start 126.865498 93.98) (end 125.51 93.98) (width 0.4) (layer "F.Cu") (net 7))
 (segment (start 126.865498 93.98) (end 126.865498 95.080498) (width 0.4) (layer "F.Cu") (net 7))
 (segment (start 130.845 99.06) (end 131.09 99.06) (width 0.4) (layer "F.Cu") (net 7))
 (segment (start 126.865498 95.080498) (end 130.845 99.06) (width 0.4) (layer "F.Cu") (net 7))
 (segment (start 137.795 81.109) (end 135.084 83.82) (width 0.4) (layer "F.Cu") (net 7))
 (segment (start 135.084 83.82) (end 134.62 83.82) (width 0.4) (layer "F.Cu") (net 7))
 (segment (start 125.51 88.9) (end 127 88.9) (width 0.4) (layer "F.Cu") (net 7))
 (via (at 127 88.9) (size 0.8) (drill 0.4) (layers "F.Cu" "B.Cu") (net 7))
 (via (at 126.865498 93.98) (size 0.8) (drill 0.4) (layers "F.Cu" "B.Cu") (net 7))
 (via (at 134.62 83.82) (size 0.8) (drill 0.4) (layers "F.Cu" "B.Cu") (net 7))
 (segment (start 132.88 85.56) (end 128.74 85.56) (width 0.4) (layer "B.Cu") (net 7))
 (segment (start 127 88.9) (end 127 93.845498) (width 0.4) (layer "B.Cu") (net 7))
 (segment (start 124.46 86.36) (end 127 88.9) (width 0.4) (layer "B.Cu") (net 7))
 (segment (start 124.46 83.82) (end 124.46 86.36) (width 0.4) (layer "B.Cu") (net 7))
 (segment (start 134.62 83.82) (end 132.88 85.56) (width 0.4) (layer "B.Cu") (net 7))
 (segment (start 128.74 85.56) (end 127 83.82) (width 0.4) (layer "B.Cu") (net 7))
 (segment (start 127 93.845498) (end 126.865498 93.98) (width 0.4) (layer "B.Cu") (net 7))
 (segment (start 127 83.82) (end 124.46 83.82) (width 0.4) (layer "B.Cu") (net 7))
 (segment (start 124.46 96.52) (end 123.41 95.47) (width 0.4) (layer "F.Cu") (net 6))
 (segment (start 123.41 95.47) (end 123.41 94.93) (width 0.4) (layer "F.Cu") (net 6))
 (segment (start 132.08 96.52) (end 133.63 96.52) (width 0.4) (layer "F.Cu") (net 6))
 (segment (start 133.63 96.52) (end 134.62 95.53) (width 0.4) (layer "F.Cu") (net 6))
 (via (at 132.08 96.52) (size 0.8) (drill 0.4) (layers "F.Cu" "B.Cu") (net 6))
 (via (at 124.46 96.52) (size 0.8) (drill 0.4) (layers "F.Cu" "B.Cu") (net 6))
 (segment (start 124.46 96.52) (end 132.08 96.52) (width 0.4) (layer "B.Cu") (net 6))
 (segment (start 127.99 99.06) (end 125.55 99.06) (width 0.4) (layer "F.Cu") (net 4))
 (segment (start 129.54 100.61) (end 127.99 99.06) (width 0.4) (layer "F.Cu") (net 4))
 (segment (start 140.335 100.965) (end 139.7 101.6) (width 0.4) (layer "F.Cu") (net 4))
 (segment (start 129.54 101.6) (end 129.54 100.61) (width 0.4) (layer "F.Cu") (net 4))
 (segment (start 140.335 86.531) (end 140.335 100.965) (width 0.4) (layer "F.Cu") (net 4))
 (via (at 139.7 101.6) (size 0.8) (drill 0.4) (layers "F.Cu" "B.Cu") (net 4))
 (via (at 129.54 101.6) (size 0.8) (drill 0.4) (layers "F.Cu" "B.Cu") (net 4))
 (segment (start 139.7 101.6) (end 129.54 101.6) (width 0.4) (layer "B.Cu") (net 4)))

